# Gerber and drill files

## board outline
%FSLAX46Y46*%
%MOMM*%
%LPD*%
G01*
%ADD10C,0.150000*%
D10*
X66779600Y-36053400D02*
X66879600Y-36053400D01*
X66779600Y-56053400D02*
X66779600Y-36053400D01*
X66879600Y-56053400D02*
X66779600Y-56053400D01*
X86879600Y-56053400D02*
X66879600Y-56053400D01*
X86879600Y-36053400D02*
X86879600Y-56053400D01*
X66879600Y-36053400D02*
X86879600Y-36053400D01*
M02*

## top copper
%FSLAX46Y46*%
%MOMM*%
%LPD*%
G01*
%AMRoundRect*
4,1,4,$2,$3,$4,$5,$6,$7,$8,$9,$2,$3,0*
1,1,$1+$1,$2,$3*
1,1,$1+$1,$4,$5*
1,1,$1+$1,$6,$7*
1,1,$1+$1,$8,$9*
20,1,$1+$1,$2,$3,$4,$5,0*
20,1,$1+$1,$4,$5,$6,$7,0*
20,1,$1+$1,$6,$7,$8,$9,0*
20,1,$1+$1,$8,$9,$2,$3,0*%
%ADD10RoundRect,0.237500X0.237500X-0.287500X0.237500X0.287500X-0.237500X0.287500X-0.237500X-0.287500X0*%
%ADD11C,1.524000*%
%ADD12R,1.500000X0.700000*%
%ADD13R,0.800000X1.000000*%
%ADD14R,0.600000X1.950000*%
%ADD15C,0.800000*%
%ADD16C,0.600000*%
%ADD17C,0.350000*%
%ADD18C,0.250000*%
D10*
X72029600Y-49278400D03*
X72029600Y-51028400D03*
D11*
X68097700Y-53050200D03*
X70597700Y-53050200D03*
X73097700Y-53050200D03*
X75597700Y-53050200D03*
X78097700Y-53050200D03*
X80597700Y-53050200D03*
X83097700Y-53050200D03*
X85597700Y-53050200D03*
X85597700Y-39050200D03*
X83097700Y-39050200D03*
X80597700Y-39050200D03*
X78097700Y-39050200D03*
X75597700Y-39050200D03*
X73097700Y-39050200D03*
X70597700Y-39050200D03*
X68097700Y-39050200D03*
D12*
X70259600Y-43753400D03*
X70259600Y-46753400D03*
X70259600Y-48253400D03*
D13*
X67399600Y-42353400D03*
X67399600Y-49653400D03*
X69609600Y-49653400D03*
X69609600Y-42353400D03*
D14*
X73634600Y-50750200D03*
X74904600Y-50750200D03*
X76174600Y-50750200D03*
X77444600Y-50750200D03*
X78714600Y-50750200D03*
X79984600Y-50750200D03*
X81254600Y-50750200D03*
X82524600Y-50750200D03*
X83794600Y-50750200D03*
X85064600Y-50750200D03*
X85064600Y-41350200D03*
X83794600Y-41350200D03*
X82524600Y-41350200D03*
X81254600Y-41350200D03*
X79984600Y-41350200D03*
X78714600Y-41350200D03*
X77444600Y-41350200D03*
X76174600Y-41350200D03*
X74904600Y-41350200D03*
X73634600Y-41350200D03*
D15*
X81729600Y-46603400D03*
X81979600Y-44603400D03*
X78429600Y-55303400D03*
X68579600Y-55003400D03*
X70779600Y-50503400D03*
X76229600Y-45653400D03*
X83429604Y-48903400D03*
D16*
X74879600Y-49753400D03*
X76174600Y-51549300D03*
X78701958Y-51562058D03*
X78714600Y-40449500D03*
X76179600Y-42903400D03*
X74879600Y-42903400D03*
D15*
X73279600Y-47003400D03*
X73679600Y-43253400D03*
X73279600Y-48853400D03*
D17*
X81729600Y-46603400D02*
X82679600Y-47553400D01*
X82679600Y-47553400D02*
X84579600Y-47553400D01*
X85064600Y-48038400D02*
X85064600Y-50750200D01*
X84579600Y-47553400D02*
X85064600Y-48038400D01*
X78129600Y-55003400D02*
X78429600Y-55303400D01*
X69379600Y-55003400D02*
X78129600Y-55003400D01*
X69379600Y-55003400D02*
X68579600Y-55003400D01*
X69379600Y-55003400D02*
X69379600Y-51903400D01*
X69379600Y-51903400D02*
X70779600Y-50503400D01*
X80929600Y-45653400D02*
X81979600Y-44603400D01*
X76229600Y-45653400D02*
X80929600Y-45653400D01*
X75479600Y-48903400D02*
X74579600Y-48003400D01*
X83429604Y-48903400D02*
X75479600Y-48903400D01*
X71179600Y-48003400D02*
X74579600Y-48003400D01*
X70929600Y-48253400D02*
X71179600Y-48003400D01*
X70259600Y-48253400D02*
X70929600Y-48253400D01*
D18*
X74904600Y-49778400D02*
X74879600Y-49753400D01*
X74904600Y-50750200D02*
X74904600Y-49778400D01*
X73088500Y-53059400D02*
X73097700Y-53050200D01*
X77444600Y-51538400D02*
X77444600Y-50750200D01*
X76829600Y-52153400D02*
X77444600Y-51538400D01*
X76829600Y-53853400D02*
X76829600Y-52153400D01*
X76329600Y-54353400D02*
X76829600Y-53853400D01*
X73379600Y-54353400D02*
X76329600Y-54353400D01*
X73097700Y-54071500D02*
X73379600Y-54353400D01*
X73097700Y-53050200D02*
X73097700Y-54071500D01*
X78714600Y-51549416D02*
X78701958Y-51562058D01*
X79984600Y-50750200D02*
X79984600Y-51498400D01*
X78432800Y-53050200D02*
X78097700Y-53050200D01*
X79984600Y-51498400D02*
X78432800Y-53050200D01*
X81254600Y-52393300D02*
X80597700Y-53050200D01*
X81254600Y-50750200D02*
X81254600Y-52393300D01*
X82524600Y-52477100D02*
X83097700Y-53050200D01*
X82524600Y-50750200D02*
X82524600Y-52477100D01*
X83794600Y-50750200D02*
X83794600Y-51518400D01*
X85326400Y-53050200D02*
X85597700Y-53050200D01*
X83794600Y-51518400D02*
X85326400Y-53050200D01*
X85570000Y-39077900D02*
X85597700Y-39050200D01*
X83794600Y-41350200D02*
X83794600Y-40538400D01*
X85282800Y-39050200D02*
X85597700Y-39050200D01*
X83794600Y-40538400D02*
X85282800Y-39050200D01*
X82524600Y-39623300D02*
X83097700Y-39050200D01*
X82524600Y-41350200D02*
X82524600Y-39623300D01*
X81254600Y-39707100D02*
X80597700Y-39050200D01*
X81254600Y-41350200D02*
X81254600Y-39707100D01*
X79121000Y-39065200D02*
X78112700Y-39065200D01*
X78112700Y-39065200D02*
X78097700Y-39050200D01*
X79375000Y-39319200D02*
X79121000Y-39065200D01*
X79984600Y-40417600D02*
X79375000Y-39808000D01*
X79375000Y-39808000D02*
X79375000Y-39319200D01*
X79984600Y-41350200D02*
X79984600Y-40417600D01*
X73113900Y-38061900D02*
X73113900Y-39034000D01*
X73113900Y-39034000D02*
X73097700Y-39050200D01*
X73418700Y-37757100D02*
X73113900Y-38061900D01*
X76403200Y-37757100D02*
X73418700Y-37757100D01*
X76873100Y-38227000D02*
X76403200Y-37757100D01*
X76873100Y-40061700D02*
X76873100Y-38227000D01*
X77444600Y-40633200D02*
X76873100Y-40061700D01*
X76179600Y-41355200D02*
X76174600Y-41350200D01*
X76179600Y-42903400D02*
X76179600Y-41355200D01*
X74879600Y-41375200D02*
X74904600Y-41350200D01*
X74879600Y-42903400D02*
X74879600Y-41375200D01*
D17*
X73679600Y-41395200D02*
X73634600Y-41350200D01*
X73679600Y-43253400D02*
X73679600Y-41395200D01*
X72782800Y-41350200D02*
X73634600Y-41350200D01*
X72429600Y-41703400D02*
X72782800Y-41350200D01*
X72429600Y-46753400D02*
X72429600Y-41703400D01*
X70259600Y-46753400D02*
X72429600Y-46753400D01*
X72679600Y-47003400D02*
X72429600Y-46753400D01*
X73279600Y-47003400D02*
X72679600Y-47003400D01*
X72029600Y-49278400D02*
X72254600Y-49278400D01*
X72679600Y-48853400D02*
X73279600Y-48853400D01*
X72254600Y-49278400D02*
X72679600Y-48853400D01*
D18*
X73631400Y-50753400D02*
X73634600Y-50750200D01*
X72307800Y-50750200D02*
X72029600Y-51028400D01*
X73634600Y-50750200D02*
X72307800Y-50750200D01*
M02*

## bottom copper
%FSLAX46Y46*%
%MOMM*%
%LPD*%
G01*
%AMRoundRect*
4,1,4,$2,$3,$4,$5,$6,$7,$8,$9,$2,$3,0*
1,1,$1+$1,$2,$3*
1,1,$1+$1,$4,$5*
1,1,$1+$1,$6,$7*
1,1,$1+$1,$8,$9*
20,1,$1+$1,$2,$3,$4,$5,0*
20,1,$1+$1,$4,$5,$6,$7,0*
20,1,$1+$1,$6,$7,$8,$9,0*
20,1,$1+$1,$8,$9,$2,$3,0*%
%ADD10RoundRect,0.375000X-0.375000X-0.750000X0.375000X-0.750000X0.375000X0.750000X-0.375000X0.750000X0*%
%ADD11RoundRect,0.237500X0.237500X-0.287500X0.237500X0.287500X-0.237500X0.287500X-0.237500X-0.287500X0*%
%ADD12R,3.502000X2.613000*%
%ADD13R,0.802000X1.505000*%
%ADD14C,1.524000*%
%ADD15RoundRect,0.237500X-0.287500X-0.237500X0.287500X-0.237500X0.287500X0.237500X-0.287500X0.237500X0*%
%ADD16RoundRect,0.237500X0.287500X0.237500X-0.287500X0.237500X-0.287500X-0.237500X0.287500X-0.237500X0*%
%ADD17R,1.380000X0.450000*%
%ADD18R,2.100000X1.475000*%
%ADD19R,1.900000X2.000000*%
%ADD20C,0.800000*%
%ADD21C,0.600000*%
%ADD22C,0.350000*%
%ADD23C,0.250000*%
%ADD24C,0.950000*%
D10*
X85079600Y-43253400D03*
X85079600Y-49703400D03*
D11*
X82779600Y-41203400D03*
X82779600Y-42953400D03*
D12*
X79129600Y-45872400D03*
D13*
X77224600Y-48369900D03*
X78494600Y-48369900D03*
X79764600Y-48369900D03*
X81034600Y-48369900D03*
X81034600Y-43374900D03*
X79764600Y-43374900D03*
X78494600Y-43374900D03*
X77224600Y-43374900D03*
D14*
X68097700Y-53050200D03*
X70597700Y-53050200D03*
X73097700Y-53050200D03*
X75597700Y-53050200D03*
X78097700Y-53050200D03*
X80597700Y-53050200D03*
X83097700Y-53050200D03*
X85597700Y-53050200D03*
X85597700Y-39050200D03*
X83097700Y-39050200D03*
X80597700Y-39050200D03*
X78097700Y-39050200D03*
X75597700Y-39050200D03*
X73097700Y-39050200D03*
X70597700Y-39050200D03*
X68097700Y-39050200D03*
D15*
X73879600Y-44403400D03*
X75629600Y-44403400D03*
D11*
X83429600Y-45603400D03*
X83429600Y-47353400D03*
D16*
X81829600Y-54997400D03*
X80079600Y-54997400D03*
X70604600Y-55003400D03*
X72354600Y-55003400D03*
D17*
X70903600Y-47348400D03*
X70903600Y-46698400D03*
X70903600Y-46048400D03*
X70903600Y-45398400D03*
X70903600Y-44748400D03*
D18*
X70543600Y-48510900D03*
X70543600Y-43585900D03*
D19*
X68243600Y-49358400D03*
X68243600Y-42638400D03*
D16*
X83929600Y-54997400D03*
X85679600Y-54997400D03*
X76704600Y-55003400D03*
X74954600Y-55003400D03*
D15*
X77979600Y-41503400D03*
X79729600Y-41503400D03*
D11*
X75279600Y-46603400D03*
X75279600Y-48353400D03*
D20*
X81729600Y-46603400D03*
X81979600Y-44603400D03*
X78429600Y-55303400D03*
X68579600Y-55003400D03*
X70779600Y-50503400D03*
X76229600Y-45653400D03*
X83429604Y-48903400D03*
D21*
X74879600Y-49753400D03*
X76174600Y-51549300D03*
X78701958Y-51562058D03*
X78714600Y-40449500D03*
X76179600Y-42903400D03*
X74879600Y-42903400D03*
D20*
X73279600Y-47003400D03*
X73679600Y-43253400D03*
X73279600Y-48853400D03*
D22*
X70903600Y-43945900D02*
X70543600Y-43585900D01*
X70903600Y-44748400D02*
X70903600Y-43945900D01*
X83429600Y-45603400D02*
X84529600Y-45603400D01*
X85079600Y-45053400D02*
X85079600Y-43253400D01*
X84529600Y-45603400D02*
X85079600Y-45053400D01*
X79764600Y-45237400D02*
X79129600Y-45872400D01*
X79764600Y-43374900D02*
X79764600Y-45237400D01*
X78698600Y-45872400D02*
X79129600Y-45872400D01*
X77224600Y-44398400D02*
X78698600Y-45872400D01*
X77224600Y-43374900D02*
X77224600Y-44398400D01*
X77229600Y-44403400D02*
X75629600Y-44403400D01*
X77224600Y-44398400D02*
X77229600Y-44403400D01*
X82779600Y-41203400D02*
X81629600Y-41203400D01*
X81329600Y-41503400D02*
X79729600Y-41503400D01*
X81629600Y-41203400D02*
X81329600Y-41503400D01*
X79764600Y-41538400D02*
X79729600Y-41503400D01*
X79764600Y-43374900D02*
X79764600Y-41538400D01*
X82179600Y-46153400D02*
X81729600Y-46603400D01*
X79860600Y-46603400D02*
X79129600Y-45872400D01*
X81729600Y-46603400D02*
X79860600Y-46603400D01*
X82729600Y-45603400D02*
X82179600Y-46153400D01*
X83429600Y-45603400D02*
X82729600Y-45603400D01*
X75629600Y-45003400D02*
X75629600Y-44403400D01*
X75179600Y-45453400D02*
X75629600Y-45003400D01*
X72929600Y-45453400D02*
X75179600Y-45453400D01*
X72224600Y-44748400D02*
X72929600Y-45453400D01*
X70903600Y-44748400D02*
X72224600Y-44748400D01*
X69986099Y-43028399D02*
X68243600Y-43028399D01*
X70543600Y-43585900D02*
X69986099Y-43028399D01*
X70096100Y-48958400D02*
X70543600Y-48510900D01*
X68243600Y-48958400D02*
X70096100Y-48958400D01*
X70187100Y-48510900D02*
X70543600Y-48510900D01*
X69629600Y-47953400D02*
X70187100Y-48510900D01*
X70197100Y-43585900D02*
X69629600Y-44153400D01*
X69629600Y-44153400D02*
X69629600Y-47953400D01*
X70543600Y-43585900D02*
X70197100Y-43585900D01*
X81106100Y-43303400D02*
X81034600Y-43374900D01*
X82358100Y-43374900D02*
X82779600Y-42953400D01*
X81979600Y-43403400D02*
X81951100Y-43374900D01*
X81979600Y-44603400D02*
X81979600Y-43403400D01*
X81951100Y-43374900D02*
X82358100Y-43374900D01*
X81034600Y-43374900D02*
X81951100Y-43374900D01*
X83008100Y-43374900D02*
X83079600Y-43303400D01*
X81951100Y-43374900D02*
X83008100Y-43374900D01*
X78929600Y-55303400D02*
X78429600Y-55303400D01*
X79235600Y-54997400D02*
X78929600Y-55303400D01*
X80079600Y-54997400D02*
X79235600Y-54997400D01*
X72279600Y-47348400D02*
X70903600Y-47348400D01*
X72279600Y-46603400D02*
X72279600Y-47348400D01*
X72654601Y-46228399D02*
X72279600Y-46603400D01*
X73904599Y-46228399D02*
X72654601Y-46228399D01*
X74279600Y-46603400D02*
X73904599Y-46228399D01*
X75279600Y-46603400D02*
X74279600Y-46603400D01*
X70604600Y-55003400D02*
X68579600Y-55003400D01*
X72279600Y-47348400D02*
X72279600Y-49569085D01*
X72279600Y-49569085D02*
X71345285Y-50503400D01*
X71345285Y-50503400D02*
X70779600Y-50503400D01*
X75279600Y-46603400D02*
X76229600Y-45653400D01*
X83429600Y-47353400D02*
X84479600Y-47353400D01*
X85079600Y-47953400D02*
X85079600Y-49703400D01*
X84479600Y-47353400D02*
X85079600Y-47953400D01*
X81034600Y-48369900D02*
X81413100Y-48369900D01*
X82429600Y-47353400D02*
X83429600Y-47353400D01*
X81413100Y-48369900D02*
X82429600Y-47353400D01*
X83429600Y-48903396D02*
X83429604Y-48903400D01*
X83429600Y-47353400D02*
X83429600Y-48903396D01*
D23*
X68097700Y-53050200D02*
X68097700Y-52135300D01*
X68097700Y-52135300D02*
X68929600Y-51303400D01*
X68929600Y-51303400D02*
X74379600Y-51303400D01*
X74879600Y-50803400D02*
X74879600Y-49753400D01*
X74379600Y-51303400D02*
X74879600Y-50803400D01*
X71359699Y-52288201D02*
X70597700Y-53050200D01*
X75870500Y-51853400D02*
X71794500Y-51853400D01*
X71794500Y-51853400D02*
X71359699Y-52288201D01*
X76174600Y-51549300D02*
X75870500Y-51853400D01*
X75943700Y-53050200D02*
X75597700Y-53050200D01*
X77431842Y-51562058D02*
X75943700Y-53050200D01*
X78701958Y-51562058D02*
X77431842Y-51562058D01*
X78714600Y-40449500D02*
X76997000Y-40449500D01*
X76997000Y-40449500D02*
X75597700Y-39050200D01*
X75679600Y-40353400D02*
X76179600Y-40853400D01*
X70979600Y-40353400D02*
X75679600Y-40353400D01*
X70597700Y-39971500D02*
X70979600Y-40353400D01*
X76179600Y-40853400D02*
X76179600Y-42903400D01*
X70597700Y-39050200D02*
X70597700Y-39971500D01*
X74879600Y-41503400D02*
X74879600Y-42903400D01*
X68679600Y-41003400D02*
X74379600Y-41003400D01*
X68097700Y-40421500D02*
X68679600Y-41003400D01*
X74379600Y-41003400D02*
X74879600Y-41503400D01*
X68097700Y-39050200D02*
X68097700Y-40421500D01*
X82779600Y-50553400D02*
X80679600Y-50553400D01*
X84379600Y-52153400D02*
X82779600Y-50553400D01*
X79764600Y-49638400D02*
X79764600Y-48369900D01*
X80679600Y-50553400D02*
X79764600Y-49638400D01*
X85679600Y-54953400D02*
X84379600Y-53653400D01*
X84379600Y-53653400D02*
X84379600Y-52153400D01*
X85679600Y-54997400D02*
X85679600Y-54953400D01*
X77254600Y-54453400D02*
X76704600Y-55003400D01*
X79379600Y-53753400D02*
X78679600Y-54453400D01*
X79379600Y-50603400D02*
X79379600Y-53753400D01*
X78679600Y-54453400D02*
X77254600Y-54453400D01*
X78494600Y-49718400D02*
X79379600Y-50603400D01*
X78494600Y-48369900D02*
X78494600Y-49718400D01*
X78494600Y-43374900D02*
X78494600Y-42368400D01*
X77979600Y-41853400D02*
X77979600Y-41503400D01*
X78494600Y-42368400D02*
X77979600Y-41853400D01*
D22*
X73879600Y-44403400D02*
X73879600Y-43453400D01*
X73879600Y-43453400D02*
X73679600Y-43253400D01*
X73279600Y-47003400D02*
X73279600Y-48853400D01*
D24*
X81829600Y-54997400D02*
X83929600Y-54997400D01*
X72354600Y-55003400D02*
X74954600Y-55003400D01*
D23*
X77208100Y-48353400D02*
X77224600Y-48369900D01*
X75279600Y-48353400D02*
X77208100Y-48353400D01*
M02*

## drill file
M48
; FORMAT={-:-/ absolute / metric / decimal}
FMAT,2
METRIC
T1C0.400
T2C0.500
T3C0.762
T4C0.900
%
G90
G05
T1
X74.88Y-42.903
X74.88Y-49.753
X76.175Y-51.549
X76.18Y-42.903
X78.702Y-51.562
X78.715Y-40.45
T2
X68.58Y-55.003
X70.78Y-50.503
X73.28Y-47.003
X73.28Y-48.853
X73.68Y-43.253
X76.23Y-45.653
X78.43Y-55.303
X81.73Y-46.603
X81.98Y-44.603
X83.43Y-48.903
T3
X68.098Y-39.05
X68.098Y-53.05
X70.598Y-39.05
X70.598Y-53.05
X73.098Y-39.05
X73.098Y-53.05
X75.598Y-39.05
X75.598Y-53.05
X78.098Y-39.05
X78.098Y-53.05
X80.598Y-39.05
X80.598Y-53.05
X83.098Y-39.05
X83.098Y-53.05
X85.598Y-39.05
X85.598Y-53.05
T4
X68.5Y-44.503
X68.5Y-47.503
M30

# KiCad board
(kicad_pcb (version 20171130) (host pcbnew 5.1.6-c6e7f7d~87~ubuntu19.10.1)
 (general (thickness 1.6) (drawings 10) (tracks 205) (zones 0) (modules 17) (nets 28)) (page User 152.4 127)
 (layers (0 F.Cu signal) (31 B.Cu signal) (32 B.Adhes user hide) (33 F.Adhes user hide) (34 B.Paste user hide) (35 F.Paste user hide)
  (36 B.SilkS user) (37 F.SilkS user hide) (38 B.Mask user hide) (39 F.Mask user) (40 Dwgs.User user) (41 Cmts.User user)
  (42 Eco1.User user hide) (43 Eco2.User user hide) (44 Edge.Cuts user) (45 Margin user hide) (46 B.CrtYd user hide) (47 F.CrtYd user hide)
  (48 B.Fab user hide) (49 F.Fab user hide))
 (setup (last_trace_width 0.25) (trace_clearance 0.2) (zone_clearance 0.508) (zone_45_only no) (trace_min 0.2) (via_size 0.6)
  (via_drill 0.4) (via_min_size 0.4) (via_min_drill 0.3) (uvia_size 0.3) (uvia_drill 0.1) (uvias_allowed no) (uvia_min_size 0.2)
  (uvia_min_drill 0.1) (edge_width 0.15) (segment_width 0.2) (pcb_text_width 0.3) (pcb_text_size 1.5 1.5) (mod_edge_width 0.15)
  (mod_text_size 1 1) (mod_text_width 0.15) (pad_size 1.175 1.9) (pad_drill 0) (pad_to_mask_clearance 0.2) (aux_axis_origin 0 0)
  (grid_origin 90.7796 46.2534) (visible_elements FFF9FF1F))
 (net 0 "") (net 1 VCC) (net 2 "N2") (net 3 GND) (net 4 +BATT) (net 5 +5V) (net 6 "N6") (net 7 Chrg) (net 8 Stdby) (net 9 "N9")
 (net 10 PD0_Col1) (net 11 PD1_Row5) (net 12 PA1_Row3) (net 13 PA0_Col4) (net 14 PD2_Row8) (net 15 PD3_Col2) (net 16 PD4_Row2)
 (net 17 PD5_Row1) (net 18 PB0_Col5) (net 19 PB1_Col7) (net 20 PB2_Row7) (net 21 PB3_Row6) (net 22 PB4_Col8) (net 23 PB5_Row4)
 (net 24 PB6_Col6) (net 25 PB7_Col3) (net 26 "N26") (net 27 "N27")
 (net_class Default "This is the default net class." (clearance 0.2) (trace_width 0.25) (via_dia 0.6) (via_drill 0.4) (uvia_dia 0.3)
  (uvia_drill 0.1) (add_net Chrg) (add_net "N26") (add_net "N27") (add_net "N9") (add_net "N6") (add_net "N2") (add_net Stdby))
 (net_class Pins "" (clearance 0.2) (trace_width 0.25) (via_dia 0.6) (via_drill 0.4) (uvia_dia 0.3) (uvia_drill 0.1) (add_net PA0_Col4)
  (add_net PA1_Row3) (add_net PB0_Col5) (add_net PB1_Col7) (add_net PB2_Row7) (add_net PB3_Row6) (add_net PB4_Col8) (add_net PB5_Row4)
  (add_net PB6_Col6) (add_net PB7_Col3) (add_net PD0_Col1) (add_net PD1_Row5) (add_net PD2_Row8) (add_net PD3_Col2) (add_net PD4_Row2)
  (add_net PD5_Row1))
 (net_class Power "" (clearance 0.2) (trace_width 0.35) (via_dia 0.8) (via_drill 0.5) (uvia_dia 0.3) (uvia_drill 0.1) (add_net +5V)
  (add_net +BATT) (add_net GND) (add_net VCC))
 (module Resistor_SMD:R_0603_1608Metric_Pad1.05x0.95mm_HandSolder (layer F.Cu) (at 72.0296 50.1534 90)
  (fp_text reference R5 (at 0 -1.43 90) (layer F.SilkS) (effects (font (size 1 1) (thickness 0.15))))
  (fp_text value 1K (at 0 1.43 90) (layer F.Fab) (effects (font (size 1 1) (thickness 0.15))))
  (pad 2 smd roundrect (at 0.875 0 90) (size 1.05 0.95) (layers F.Cu F.Paste F.Mask) (roundrect_rratio 0.25) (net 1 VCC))
  (pad 1 smd roundrect (at -0.875 0 90) (size 1.05 0.95) (layers F.Cu F.Paste F.Mask) (roundrect_rratio 0.25) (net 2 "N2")))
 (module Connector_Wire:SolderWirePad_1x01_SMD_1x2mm (layer B.Cu) (at 85.0796 43.2534)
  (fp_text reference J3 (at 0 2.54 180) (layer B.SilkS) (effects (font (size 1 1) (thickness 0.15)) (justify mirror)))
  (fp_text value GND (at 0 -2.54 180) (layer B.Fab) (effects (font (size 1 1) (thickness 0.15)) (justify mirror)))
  (pad 1 smd roundrect (at 0 0) (size 1.5 2.25) (layers B.Cu B.Paste B.Mask) (roundrect_rratio 0.25) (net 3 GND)))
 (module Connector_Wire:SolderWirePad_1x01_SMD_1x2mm (layer B.Cu) (at 85.0796 49.7034)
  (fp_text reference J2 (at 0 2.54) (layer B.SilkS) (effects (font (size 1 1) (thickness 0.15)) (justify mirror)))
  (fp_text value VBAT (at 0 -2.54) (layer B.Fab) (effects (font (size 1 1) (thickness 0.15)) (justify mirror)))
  (pad 1 smd roundrect (at 0 0) (size 1.5 2.25) (layers B.Cu B.Paste B.Mask) (roundrect_rratio 0.25) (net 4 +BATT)))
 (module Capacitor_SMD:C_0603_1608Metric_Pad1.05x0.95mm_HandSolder (layer B.Cu) (at 82.7796 42.0784 90)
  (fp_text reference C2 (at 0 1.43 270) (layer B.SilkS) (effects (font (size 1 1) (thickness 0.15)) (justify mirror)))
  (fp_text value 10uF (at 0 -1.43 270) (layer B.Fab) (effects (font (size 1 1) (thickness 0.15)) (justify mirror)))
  (pad 2 smd roundrect (at 0.875 0 90) (size 1.05 0.95) (layers B.Cu B.Paste B.Mask) (roundrect_rratio 0.25) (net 3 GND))
  (pad 1 smd roundrect (at -0.875 0 90) (size 1.05 0.95) (layers B.Cu B.Paste B.Mask) (roundrect_rratio 0.25) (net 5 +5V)))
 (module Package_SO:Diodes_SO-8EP (layer B.Cu) (at 79.1296 45.8724 270)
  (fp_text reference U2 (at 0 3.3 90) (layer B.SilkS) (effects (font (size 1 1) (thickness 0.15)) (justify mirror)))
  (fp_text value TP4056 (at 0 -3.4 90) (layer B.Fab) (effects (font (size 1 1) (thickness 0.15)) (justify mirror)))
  (pad 9 smd rect (at 0 0 270) (size 2.613 3.502) (layers B.Cu B.Paste B.Mask) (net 3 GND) (solder_paste_margin_ratio -0.2))
  (pad 8 smd rect (at 2.4975 1.905 270) (size 1.505 0.802) (layers B.Cu B.Paste B.Mask) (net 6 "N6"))
  (pad 7 smd rect (at 2.4975 0.635 270) (size 1.505 0.802) (layers B.Cu B.Paste B.Mask) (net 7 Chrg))
  (pad 6 smd rect (at 2.4975 -0.635 270) (size 1.505 0.802) (layers B.Cu B.Paste B.Mask) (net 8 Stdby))
  (pad 5 smd rect (at 2.4975 -1.905 270) (size 1.505 0.802) (layers B.Cu B.Paste B.Mask) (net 4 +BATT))
  (pad 4 smd rect (at -2.4975 -1.905 270) (size 1.505 0.802) (layers B.Cu B.Paste B.Mask) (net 5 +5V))
  (pad 3 smd rect (at -2.4975 -0.635 270) (size 1.505 0.802) (layers B.Cu B.Paste B.Mask) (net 3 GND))
  (pad 2 smd rect (at -2.4975 0.635 270) (size 1.505 0.802) (layers B.Cu B.Paste B.Mask) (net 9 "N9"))
  (pad 1 smd rect (at -2.4975 1.905 270) (size 1.505 0.802) (layers B.Cu B.Paste B.Mask) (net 3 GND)))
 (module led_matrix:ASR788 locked (layer F.Cu) (at 76.8477 46.0502)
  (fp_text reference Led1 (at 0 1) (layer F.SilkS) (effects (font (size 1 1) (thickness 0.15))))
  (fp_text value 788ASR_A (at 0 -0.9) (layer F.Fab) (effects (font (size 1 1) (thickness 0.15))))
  (pad 1 thru_hole circle (at -8.75 7) (size 1.524 1.524) (drill 0.762) (layers *.Cu *.Mask) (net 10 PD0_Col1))
  (pad 2 thru_hole circle (at -6.25 7) (size 1.524 1.524) (drill 0.762) (layers *.Cu *.Mask) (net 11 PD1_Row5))
  (pad 3 thru_hole circle (at -3.75 7) (size 1.524 1.524) (drill 0.762) (layers *.Cu *.Mask) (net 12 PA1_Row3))
  (pad 4 thru_hole circle (at -1.25 7) (size 1.524 1.524) (drill 0.762) (layers *.Cu *.Mask) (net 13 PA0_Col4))
  (pad 5 thru_hole circle (at 1.25 7) (size 1.524 1.524) (drill 0.762) (layers *.Cu *.Mask) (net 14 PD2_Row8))
  (pad 6 thru_hole circle (at 3.75 7) (size 1.524 1.524) (drill 0.762) (layers *.Cu *.Mask) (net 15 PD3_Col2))
  (pad 7 thru_hole circle (at 6.25 7) (size 1.524 1.524) (drill 0.762) (layers *.Cu *.Mask) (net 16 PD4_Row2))
  (pad 8 thru_hole circle (at 8.75 7) (size 1.524 1.524) (drill 0.762) (layers *.Cu *.Mask) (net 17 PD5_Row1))
  (pad 9 thru_hole circle (at 8.75 -7) (size 1.524 1.524) (drill 0.762) (layers *.Cu *.Mask) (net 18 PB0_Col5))
  (pad 10 thru_hole circle (at 6.25 -7) (size 1.524 1.524) (drill 0.762) (layers *.Cu *.Mask) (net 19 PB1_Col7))
  (pad 11 thru_hole circle (at 3.75 -7) (size 1.524 1.524) (drill 0.762) (layers *.Cu *.Mask) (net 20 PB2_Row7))
  (pad 12 thru_hole circle (at 1.25 -7) (size 1.524 1.524) (drill 0.762) (layers *.Cu *.Mask) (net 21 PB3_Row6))
  (pad 13 thru_hole circle (at -1.25 -7) (size 1.524 1.524) (drill 0.762) (layers *.Cu *.Mask) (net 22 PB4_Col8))
  (pad 14 thru_hole circle (at -3.75 -7) (size 1.524 1.524) (drill 0.762) (layers *.Cu *.Mask) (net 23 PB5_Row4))
  (pad 15 thru_hole circle (at -6.25 -7) (size 1.524 1.524) (drill 0.762) (layers *.Cu *.Mask) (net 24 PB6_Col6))
  (pad 16 thru_hole circle (at -8.75 -7) (size 1.524 1.524) (drill 0.762) (layers *.Cu *.Mask) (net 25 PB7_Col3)))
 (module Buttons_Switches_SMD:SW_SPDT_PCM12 (layer F.Cu) (at 68.8296 46.0034 270)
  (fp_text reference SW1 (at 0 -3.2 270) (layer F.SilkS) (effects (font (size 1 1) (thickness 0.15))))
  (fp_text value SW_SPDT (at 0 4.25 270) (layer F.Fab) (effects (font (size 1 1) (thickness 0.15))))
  (pad "" np_thru_hole circle (at -1.5 0.33 270) (size 0.9 0.9) (drill 0.9) (layers *.Cu *.Mask))
  (pad "" np_thru_hole circle (at 1.5 0.33 270) (size 0.9 0.9) (drill 0.9) (layers *.Cu *.Mask))
  (pad 1 smd rect (at -2.25 -1.43 270) (size 0.7 1.5) (layers F.Cu F.Paste F.Mask))
  (pad 2 smd rect (at 0.75 -1.43 270) (size 0.7 1.5) (layers F.Cu F.Paste F.Mask) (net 1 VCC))
  (pad 3 smd rect (at 2.25 -1.43 270) (size 0.7 1.5) (layers F.Cu F.Paste F.Mask) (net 4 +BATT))
  (pad "" smd rect (at -3.65 1.43 270) (size 1 0.8) (layers F.Cu F.Paste F.Mask))
  (pad "" smd rect (at 3.65 1.43 270) (size 1 0.8) (layers F.Cu F.Paste F.Mask))
  (pad "" smd rect (at 3.65 -0.78 270) (size 1 0.8) (layers F.Cu F.Paste F.Mask))
  (pad "" smd rect (at -3.65 -0.78 270) (size 1 0.8) (layers F.Cu F.Paste F.Mask)))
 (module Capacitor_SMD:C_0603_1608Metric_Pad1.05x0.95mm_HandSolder (layer B.Cu) (at 74.7546 44.4034)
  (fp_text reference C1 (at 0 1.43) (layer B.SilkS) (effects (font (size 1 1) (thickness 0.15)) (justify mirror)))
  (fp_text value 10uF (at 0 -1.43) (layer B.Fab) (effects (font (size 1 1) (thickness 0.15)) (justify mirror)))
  (pad 1 smd roundrect (at -0.875 0) (size 1.05 0.95) (layers B.Cu B.Paste B.Mask) (roundrect_rratio 0.25) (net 1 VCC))
  (pad 2 smd roundrect (at 0.875 0) (size 1.05 0.95) (layers B.Cu B.Paste B.Mask) (roundrect_rratio 0.25) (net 3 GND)))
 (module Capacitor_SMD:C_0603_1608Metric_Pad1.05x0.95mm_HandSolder (layer B.Cu) (at 83.4296 46.4784 90)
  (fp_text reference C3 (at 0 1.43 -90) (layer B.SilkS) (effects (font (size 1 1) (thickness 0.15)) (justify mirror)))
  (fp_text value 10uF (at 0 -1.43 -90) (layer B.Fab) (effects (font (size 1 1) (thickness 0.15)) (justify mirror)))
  (pad 2 smd roundrect (at 0.875 0 90) (size 1.05 0.95) (layers B.Cu B.Paste B.Mask) (roundrect_rratio 0.25) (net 3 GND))
  (pad 1 smd roundrect (at -0.875 0 90) (size 1.05 0.95) (layers B.Cu B.Paste B.Mask) (roundrect_rratio 0.25) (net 4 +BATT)))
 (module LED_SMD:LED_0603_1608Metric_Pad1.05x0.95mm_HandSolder (layer B.Cu) (at 80.9546 54.9974 180)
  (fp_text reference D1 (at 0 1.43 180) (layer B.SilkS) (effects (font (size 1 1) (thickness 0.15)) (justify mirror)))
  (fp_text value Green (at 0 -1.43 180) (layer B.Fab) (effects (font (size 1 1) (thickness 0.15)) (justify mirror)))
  (pad 1 smd roundrect (at -0.875 0 180) (size 1.05 0.95) (layers B.Cu B.Paste B.Mask) (roundrect_rratio 0.25) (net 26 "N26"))
  (pad 2 smd roundrect (at 0.875 0 180) (size 1.05 0.95) (layers B.Cu B.Paste B.Mask) (roundrect_rratio 0.25) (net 5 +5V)))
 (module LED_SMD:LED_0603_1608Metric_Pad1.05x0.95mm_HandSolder (layer B.Cu) (at 71.4796 55.0034 180)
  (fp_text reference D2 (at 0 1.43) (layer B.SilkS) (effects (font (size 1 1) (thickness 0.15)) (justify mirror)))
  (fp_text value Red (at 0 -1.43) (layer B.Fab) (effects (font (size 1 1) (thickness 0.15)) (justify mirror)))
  (pad 2 smd roundrect (at 0.875 0 180) (size 1.05 0.95) (layers B.Cu B.Paste B.Mask) (roundrect_rratio 0.25) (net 5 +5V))
  (pad 1 smd roundrect (at -0.875 0 180) (size 1.05 0.95) (layers B.Cu B.Paste B.Mask) (roundrect_rratio 0.25) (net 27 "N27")))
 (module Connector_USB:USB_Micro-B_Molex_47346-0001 (layer B.Cu) (at 69.4436 46.0484 90)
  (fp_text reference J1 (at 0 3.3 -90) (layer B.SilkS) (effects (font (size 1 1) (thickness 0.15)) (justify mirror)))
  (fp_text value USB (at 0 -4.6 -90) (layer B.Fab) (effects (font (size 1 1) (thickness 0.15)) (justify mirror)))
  (pad 1 smd rect (at -1.3 1.46 90) (size 0.45 1.38) (layers B.Cu B.Paste B.Mask) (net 5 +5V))
  (pad 2 smd rect (at -0.65 1.46 90) (size 0.45 1.38) (layers B.Cu B.Paste B.Mask))
  (pad 3 smd rect (at 0 1.46 90) (size 0.45 1.38) (layers B.Cu B.Paste B.Mask))
  (pad 4 smd rect (at 0.65 1.46 90) (size 0.45 1.38) (layers B.Cu B.Paste B.Mask))
  (pad 5 smd rect (at 1.3 1.46 90) (size 0.45 1.38) (layers B.Cu B.Paste B.Mask) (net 3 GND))
  (pad 6 smd rect (at -2.4625 1.1 90) (size 1.475 2.1) (layers B.Cu B.Paste B.Mask) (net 3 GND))
  (pad 6 smd rect (at 2.4625 1.1 90) (size 1.475 2.1) (layers B.Cu B.Paste B.Mask) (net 3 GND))
  (pad 6 smd rect (at -3.31 -1.2 90) (size 2 1.9) (layers B.Cu B.Paste B.Mask) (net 3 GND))
  (pad 6 smd rect (at 3.41 -1.2 90) (size 2 1.9) (layers B.Cu B.Paste B.Mask) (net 3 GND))
  (pad 6 smd rect (at -0.84 -1.2 90) (size 1.175 1.9) (layers Eco1.User))
  (pad 6 smd rect (at 0.84 -1.2 90) (size 1.175 1.9) (layers Eco1.User)))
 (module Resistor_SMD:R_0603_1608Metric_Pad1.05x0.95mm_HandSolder (layer B.Cu) (at 84.8046 54.9974 180)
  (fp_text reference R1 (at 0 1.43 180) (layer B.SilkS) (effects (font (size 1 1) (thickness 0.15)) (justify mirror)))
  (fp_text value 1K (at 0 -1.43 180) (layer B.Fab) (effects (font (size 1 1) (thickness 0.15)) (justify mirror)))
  (pad 2 smd roundrect (at 0.875 0 180) (size 1.05 0.95) (layers B.Cu B.Paste B.Mask) (roundrect_rratio 0.25) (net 26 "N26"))
  (pad 1 smd roundrect (at -0.875 0 180) (size 1.05 0.95) (layers B.Cu B.Paste B.Mask) (roundrect_rratio 0.25) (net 8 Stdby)))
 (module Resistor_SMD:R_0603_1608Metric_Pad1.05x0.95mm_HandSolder (layer B.Cu) (at 75.8296 55.0034 180)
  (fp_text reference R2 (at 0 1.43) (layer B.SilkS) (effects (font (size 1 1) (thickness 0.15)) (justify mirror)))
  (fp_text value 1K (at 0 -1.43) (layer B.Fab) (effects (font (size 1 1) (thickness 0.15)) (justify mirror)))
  (pad 1 smd roundrect (at -0.875 0 180) (size 1.05 0.95) (layers B.Cu B.Paste B.Mask) (roundrect_rratio 0.25) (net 7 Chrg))
  (pad 2 smd roundrect (at 0.875 0 180) (size 1.05 0.95) (layers B.Cu B.Paste B.Mask) (roundrect_rratio 0.25) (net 27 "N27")))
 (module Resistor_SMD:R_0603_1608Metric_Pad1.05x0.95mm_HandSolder (layer B.Cu) (at 78.8546 41.5034)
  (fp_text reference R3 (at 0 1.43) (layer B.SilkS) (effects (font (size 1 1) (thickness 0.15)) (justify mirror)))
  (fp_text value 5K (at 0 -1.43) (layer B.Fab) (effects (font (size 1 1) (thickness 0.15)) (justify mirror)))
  (pad 1 smd roundrect (at -0.875 0) (size 1.05 0.95) (layers B.Cu B.Paste B.Mask) (roundrect_rratio 0.25) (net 9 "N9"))
  (pad 2 smd roundrect (at 0.875 0) (size 1.05 0.95) (layers B.Cu B.Paste B.Mask) (roundrect_rratio 0.25) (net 3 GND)))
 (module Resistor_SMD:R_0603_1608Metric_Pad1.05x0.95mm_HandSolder (layer B.Cu) (at 75.2796 47.4784 90)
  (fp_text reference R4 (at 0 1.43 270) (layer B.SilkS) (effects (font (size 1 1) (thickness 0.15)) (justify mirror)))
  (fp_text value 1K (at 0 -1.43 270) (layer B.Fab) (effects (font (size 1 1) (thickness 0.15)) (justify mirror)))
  (pad 2 smd roundrect (at 0.875 0 90) (size 1.05 0.95) (layers B.Cu B.Paste B.Mask) (roundrect_rratio 0.25) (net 5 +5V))
  (pad 1 smd roundrect (at -0.875 0 90) (size 1.05 0.95) (layers B.Cu B.Paste B.Mask) (roundrect_rratio 0.25) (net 6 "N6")))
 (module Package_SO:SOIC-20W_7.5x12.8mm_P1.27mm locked (layer F.Cu) (at 79.3496 46.0502 90)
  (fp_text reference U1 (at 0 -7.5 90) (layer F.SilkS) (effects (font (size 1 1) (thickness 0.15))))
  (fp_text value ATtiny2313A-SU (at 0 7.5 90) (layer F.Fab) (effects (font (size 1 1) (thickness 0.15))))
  (pad 1 smd rect (at -4.7 -5.715 90) (size 1.95 0.6) (layers F.Cu F.Paste F.Mask) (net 2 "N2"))
  (pad 2 smd rect (at -4.7 -4.445 90) (size 1.95 0.6) (layers F.Cu F.Paste F.Mask) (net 10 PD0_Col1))
  (pad 3 smd rect (at -4.7 -3.175 90) (size 1.95 0.6) (layers F.Cu F.Paste F.Mask) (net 11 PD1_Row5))
  (pad 4 smd rect (at -4.7 -1.905 90) (size 1.95 0.6) (layers F.Cu F.Paste F.Mask) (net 12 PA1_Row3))
  (pad 5 smd rect (at -4.7 -0.635 90) (size 1.95 0.6) (layers F.Cu F.Paste F.Mask) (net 13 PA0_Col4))
  (pad 6 smd rect (at -4.7 0.635 90) (size 1.95 0.6) (layers F.Cu F.Paste F.Mask) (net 14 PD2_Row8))
  (pad 7 smd rect (at -4.7 1.905 90) (size 1.95 0.6) (layers F.Cu F.Paste F.Mask) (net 15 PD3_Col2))
  (pad 8 smd rect (at -4.7 3.175 90) (size 1.95 0.6) (layers F.Cu F.Paste F.Mask) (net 16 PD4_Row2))
  (pad 9 smd rect (at -4.7 4.445 90) (size 1.95 0.6) (layers F.Cu F.Paste F.Mask) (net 17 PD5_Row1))
  (pad 10 smd rect (at -4.7 5.715 90) (size 1.95 0.6) (layers F.Cu F.Paste F.Mask) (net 3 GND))
  (pad 11 smd rect (at 4.7 5.715 90) (size 1.95 0.6) (layers F.Cu F.Paste F.Mask))
  (pad 12 smd rect (at 4.7 4.445 90) (size 1.95 0.6) (layers F.Cu F.Paste F.Mask) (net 18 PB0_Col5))
  (pad 13 smd rect (at 4.7 3.175 90) (size 1.95 0.6) (layers F.Cu F.Paste F.Mask) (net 19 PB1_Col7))
  (pad 14 smd rect (at 4.7 1.905 90) (size 1.95 0.6) (layers F.Cu F.Paste F.Mask) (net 20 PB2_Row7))
  (pad 15 smd rect (at 4.7 0.635 90) (size 1.95 0.6) (layers F.Cu F.Paste F.Mask) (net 21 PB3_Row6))
  (pad 16 smd rect (at 4.7 -0.635 90) (size 1.95 0.6) (layers F.Cu F.Paste F.Mask) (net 22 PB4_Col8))
  (pad 17 smd rect (at 4.7 -1.905 90) (size 1.95 0.6) (layers F.Cu F.Paste F.Mask) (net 23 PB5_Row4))
  (pad 18 smd rect (at 4.7 -3.175 90) (size 1.95 0.6) (layers F.Cu F.Paste F.Mask) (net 24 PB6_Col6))
  (pad 19 smd rect (at 4.7 -4.445 90) (size 1.95 0.6) (layers F.Cu F.Paste F.Mask) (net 25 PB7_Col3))
  (pad 20 smd rect (at 4.7 -5.715 90) (size 1.95 0.6) (layers F.Cu F.Paste F.Mask) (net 1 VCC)))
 (gr_line (start 66.7796 36.0534) (end 66.8796 36.0534) (layer Edge.Cuts) (width 0.15))
 (gr_line (start 66.7796 56.0534) (end 66.7796 36.0534) (layer Edge.Cuts) (width 0.15))
 (gr_line (start 66.8796 56.0534) (end 66.7796 56.0534) (layer Edge.Cuts) (width 0.15))
 (gr_line (start 86.8796 56.0534) (end 66.8796 56.0534) (layer Edge.Cuts) (width 0.15))
 (gr_line (start 86.8796 36.0534) (end 86.8796 56.0534) (layer Edge.Cuts) (width 0.15))
 (gr_line (start 66.8796 36.0534) (end 86.8796 36.0534) (layer Edge.Cuts) (width 0.15))
 (segment (start 70.9036 43.9459) (end 70.5436 43.5859) (width 0.35) (layer B.Cu) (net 3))
 (segment (start 70.9036 44.7484) (end 70.9036 43.9459) (width 0.35) (layer B.Cu) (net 3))
 (segment (start 83.4296 45.6034) (end 84.5296 45.6034) (width 0.35) (layer B.Cu) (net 3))
 (segment (start 85.0796 45.0534) (end 85.0796 43.2534) (width 0.35) (layer B.Cu) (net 3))
 (segment (start 84.5296 45.6034) (end 85.0796 45.0534) (width 0.35) (layer B.Cu) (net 3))
 (segment (start 79.7646 45.2374) (end 79.1296 45.8724) (width 0.35) (layer B.Cu) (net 3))
 (segment (start 79.7646 43.3749) (end 79.7646 45.2374) (width 0.35) (layer B.Cu) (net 3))
 (segment (start 78.6986 45.8724) (end 79.1296 45.8724) (width 0.35) (layer B.Cu) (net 3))
 (segment (start 77.2246 44.3984) (end 78.6986 45.8724) (width 0.35) (layer B.Cu) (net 3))
 (segment (start 77.2246 43.3749) (end 77.2246 44.3984) (width 0.35) (layer B.Cu) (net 3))
 (segment (start 77.2296 44.4034) (end 75.6296 44.4034) (width 0.35) (layer B.Cu) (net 3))
 (segment (start 77.2246 44.3984) (end 77.2296 44.4034) (width 0.35) (layer B.Cu) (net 3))
 (segment (start 82.7796 41.2034) (end 81.6296 41.2034) (width 0.35) (layer B.Cu) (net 3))
 (segment (start 81.3296 41.5034) (end 79.7296 41.5034) (width 0.35) (layer B.Cu) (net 3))
 (segment (start 81.6296 41.2034) (end 81.3296 41.5034) (width 0.35) (layer B.Cu) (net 3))
 (segment (start 79.7646 41.5384) (end 79.7296 41.5034) (width 0.35) (layer B.Cu) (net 3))
 (segment (start 79.7646 43.3749) (end 79.7646 41.5384) (width 0.35) (layer B.Cu) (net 3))
 (segment (start 82.1796 46.1534) (end 81.7296 46.6034) (width 0.35) (layer B.Cu) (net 3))
 (segment (start 79.8606 46.6034) (end 79.1296 45.8724) (width 0.35) (layer B.Cu) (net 3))
 (segment (start 81.7296 46.6034) (end 79.8606 46.6034) (width 0.35) (layer B.Cu) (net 3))
 (segment (start 82.7296 45.6034) (end 82.1796 46.1534) (width 0.35) (layer B.Cu) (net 3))
 (segment (start 83.4296 45.6034) (end 82.7296 45.6034) (width 0.35) (layer B.Cu) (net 3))
 (segment (start 75.6296 45.0034) (end 75.6296 44.4034) (width 0.35) (layer B.Cu) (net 3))
 (segment (start 75.1796 45.4534) (end 75.6296 45.0034) (width 0.35) (layer B.Cu) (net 3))
 (segment (start 72.9296 45.4534) (end 75.1796 45.4534) (width 0.35) (layer B.Cu) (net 3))
 (segment (start 72.2246 44.7484) (end 72.9296 45.4534) (width 0.35) (layer B.Cu) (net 3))
 (segment (start 70.9036 44.7484) (end 72.2246 44.7484) (width 0.35) (layer B.Cu) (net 3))
 (segment (start 69.986099 43.028399) (end 68.2436 43.028399) (width 0.35) (layer B.Cu) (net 3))
 (segment (start 70.5436 43.5859) (end 69.986099 43.028399) (width 0.35) (layer B.Cu) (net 3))
 (segment (start 70.0961 48.9584) (end 70.5436 48.5109) (width 0.35) (layer B.Cu) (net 3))
 (segment (start 68.2436 48.9584) (end 70.0961 48.9584) (width 0.35) (layer B.Cu) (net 3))
 (segment (start 70.1871 48.5109) (end 70.5436 48.5109) (width 0.35) (layer B.Cu) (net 3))
 (segment (start 69.6296 47.9534) (end 70.1871 48.5109) (width 0.35) (layer B.Cu) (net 3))
 (segment (start 70.1971 43.5859) (end 69.6296 44.1534) (width 0.35) (layer B.Cu) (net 3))
 (segment (start 69.6296 44.1534) (end 69.6296 47.9534) (width 0.35) (layer B.Cu) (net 3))
 (segment (start 70.5436 43.5859) (end 70.1971 43.5859) (width 0.35) (layer B.Cu) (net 3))
 (via (at 81.7296 46.6034) (size 0.8) (drill 0.5) (layers F.Cu B.Cu) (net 3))
 (segment (start 81.7296 46.6034) (end 82.6796 47.5534) (width 0.35) (layer F.Cu) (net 3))
 (segment (start 82.6796 47.5534) (end 84.5796 47.5534) (width 0.35) (layer F.Cu) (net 3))
 (segment (start 85.0646 48.0384) (end 85.0646 50.7502) (width 0.35) (layer F.Cu) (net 3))
 (segment (start 84.5796 47.5534) (end 85.0646 48.0384) (width 0.35) (layer F.Cu) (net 3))
 (segment (start 81.1061 43.3034) (end 81.0346 43.3749) (width 0.35) (layer B.Cu) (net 5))
 (via (at 81.9796 44.6034) (size 0.8) (drill 0.5) (layers F.Cu B.Cu) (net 5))
 (segment (start 82.3581 43.3749) (end 82.7796 42.9534) (width 0.35) (layer B.Cu) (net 5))
 (segment (start 81.9796 43.4034) (end 81.9511 43.3749) (width 0.35) (layer B.Cu) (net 5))
 (segment (start 81.9796 44.6034) (end 81.9796 43.4034) (width 0.35) (layer B.Cu) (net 5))
 (segment (start 81.9511 43.3749) (end 82.3581 43.3749) (width 0.35) (layer B.Cu) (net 5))
 (segment (start 81.0346 43.3749) (end 81.9511 43.3749) (width 0.35) (layer B.Cu) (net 5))
 (segment (start 83.0081 43.3749) (end 83.0796 43.3034) (width 0.35) (layer B.Cu) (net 5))
 (segment (start 81.9511 43.3749) (end 83.0081 43.3749) (width 0.35) (layer B.Cu) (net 5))
 (via (at 78.4296 55.3034) (size 0.8) (drill 0.5) (layers F.Cu B.Cu) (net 5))
 (via (at 68.5796 55.0034) (size 0.8) (drill 0.5) (layers F.Cu B.Cu) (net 5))
 (segment (start 78.9296 55.3034) (end 78.4296 55.3034) (width 0.35) (layer B.Cu) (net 5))
 (segment (start 79.2356 54.9974) (end 78.9296 55.3034) (width 0.35) (layer B.Cu) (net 5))
 (segment (start 80.0796 54.9974) (end 79.2356 54.9974) (width 0.35) (layer B.Cu) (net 5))
 (segment (start 72.2796 47.3484) (end 70.9036 47.3484) (width 0.35) (layer B.Cu) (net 5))
 (segment (start 72.2796 46.6034) (end 72.2796 47.3484) (width 0.35) (layer B.Cu) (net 5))
 (segment (start 72.654601 46.228399) (end 72.2796 46.6034) (width 0.35) (layer B.Cu) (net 5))
 (segment (start 73.904599 46.228399) (end 72.654601 46.228399) (width 0.35) (layer B.Cu) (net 5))
 (segment (start 74.2796 46.6034) (end 73.904599 46.228399) (width 0.35) (layer B.Cu) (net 5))
 (segment (start 75.2796 46.6034) (end 74.2796 46.6034) (width 0.35) (layer B.Cu) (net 5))
 (segment (start 78.1296 55.0034) (end 78.4296 55.3034) (width 0.35) (layer F.Cu) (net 5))
 (segment (start 69.3796 55.0034) (end 78.1296 55.0034) (width 0.35) (layer F.Cu) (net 5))
 (segment (start 70.6046 55.0034) (end 68.5796 55.0034) (width 0.35) (layer B.Cu) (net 5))
 (segment (start 69.3796 55.0034) (end 68.5796 55.0034) (width 0.35) (layer F.Cu) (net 5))
 (via (at 70.7796 50.5034) (size 0.8) (drill 0.5) (layers F.Cu B.Cu) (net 5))
 (segment (start 72.2796 47.3484) (end 72.2796 49.569085) (width 0.35) (layer B.Cu) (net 5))
 (segment (start 72.2796 49.569085) (end 71.345285 50.5034) (width 0.35) (layer B.Cu) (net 5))
 (segment (start 71.345285 50.5034) (end 70.7796 50.5034) (width 0.35) (layer B.Cu) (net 5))
 (segment (start 69.3796 55.0034) (end 69.3796 51.9034) (width 0.35) (layer F.Cu) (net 5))
 (segment (start 69.3796 51.9034) (end 70.7796 50.5034) (width 0.35) (layer F.Cu) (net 5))
 (segment (start 75.2796 46.6034) (end 76.2296 45.6534) (width 0.35) (layer B.Cu) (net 5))
 (via (at 76.2296 45.6534) (size 0.8) (drill 0.5) (layers F.Cu B.Cu) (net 5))
 (segment (start 80.9296 45.6534) (end 81.9796 44.6034) (width 0.35) (layer F.Cu) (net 5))
 (segment (start 76.2296 45.6534) (end 80.9296 45.6534) (width 0.35) (layer F.Cu) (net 5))
 (segment (start 83.4296 47.3534) (end 84.4796 47.3534) (width 0.35) (layer B.Cu) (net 4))
 (segment (start 85.0796 47.9534) (end 85.0796 49.7034) (width 0.35) (layer B.Cu) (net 4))
 (segment (start 84.4796 47.3534) (end 85.0796 47.9534) (width 0.35) (layer B.Cu) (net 4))
 (segment (start 81.0346 48.3699) (end 81.4131 48.3699) (width 0.35) (layer B.Cu) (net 4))
 (segment (start 82.4296 47.3534) (end 83.4296 47.3534) (width 0.35) (layer B.Cu) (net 4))
 (segment (start 81.4131 48.3699) (end 82.4296 47.3534) (width 0.35) (layer B.Cu) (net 4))
 (segment (start 83.4296 48.903396) (end 83.429604 48.9034) (width 0.35) (layer B.Cu) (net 4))
 (segment (start 83.4296 47.3534) (end 83.4296 48.903396) (width 0.35) (layer B.Cu) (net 4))
 (via (at 83.429604 48.9034) (size 0.8) (drill 0.5) (layers F.Cu B.Cu) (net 4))
 (segment (start 75.4796 48.9034) (end 74.5796 48.0034) (width 0.35) (layer F.Cu) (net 4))
 (segment (start 83.429604 48.9034) (end 75.4796 48.9034) (width 0.35) (layer F.Cu) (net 4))
 (segment (start 71.1796 48.0034) (end 74.5796 48.0034) (width 0.35) (layer F.Cu) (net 4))
 (segment (start 70.9296 48.2534) (end 71.1796 48.0034) (width 0.35) (layer F.Cu) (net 4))
 (segment (start 70.2596 48.2534) (end 70.9296 48.2534) (width 0.35) (layer F.Cu) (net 4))
 (via (at 74.8796 49.7534) (size 0.6) (drill 0.4) (layers F.Cu B.Cu) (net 10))
 (segment (start 74.9046 49.7784) (end 74.8796 49.7534) (width 0.25) (layer F.Cu) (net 10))
 (segment (start 74.9046 50.7502) (end 74.9046 49.7784) (width 0.25) (layer F.Cu) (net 10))
 (segment (start 68.0977 53.0502) (end 68.0977 52.1353) (width 0.25) (layer B.Cu) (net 10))
 (segment (start 68.0977 52.1353) (end 68.9296 51.3034) (width 0.25) (layer B.Cu) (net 10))
 (segment (start 68.9296 51.3034) (end 74.3796 51.3034) (width 0.25) (layer B.Cu) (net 10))
 (segment (start 74.8796 50.8034) (end 74.8796 49.7534) (width 0.25) (layer B.Cu) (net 10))
 (segment (start 74.3796 51.3034) (end 74.8796 50.8034) (width 0.25) (layer B.Cu) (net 10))
 (via (at 76.1746 51.5493) (size 0.6) (drill 0.4) (layers F.Cu B.Cu) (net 11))
 (segment (start 71.359699 52.288201) (end 70.5977 53.0502) (width 0.25) (layer B.Cu) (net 11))
 (segment (start 75.8705 51.8534) (end 71.7945 51.8534) (width 0.25) (layer B.Cu) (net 11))
 (segment (start 71.7945 51.8534) (end 71.359699 52.288201) (width 0.25) (layer B.Cu) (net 11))
 (segment (start 76.1746 51.5493) (end 75.8705 51.8534) (width 0.25) (layer B.Cu) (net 11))
 (segment (start 73.0885 53.0594) (end 73.0977 53.0502) (width 0.25) (layer F.Cu) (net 12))
 (segment (start 77.4446 51.5384) (end 77.4446 50.7502) (width 0.25) (layer F.Cu) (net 12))
 (segment (start 76.8296 52.1534) (end 77.4446 51.5384) (width 0.25) (layer F.Cu) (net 12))
 (segment (start 76.8296 53.8534) (end 76.8296 52.1534) (width 0.25) (layer F.Cu) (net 12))
 (segment (start 76.3296 54.3534) (end 76.8296 53.8534) (width 0.25) (layer F.Cu) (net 12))
 (segment (start 73.3796 54.3534) (end 76.3296 54.3534) (width 0.25) (layer F.Cu) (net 12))
 (segment (start 73.0977 54.0715) (end 73.3796 54.3534) (width 0.25) (layer F.Cu) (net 12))
 (segment (start 73.0977 53.0502) (end 73.0977 54.0715) (width 0.25) (layer F.Cu) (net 12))
 (segment (start 78.7146 51.549416) (end 78.701958 51.562058) (width 0.25) (layer F.Cu) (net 13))
 (via (at 78.701958 51.562058) (size 0.6) (drill 0.4) (layers F.Cu B.Cu) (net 13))
 (segment (start 75.9437 53.0502) (end 75.5977 53.0502) (width 0.25) (layer B.Cu) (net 13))
 (segment (start 77.431842 51.562058) (end 75.9437 53.0502) (width 0.25) (layer B.Cu) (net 13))
 (segment (start 78.701958 51.562058) (end 77.431842 51.562058) (width 0.25) (layer B.Cu) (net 13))
 (segment (start 79.9846 50.7502) (end 79.9846 51.4984) (width 0.25) (layer F.Cu) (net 14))
 (segment (start 78.4328 53.0502) (end 78.0977 53.0502) (width 0.25) (layer F.Cu) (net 14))
 (segment (start 79.9846 51.4984) (end 78.4328 53.0502) (width 0.25) (layer F.Cu) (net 14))
 (segment (start 81.2546 52.3933) (end 80.5977 53.0502) (width 0.25) (layer F.Cu) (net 15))
 (segment (start 81.2546 50.7502) (end 81.2546 52.3933) (width 0.25) (layer F.Cu) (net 15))
 (segment (start 82.5246 52.4771) (end 83.0977 53.0502) (width 0.25) (layer F.Cu) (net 16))
 (segment (start 82.5246 50.7502) (end 82.5246 52.4771) (width 0.25) (layer F.Cu) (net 16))
 (segment (start 83.7946 50.7502) (end 83.7946 51.5184) (width 0.25) (layer F.Cu) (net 17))
 (segment (start 85.3264 53.0502) (end 85.5977 53.0502) (width 0.25) (layer F.Cu) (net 17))
 (segment (start 83.7946 51.5184) (end 85.3264 53.0502) (width 0.25) (layer F.Cu) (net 17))
 (segment (start 85.57 39.0779) (end 85.5977 39.0502) (width 0.25) (layer F.Cu) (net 18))
 (segment (start 83.7946 41.3502) (end 83.7946 40.5384) (width 0.25) (layer F.Cu) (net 18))
 (segment (start 85.2828 39.0502) (end 85.5977 39.0502) (width 0.25) (layer F.Cu) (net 18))
 (segment (start 83.7946 40.5384) (end 85.2828 39.0502) (width 0.25) (layer F.Cu) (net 18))
 (segment (start 82.5246 39.6233) (end 83.0977 39.0502) (width 0.25) (layer F.Cu) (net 19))
 (segment (start 82.5246 41.3502) (end 82.5246 39.6233) (width 0.25) (layer F.Cu) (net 19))
 (segment (start 81.2546 39.7071) (end 80.5977 39.0502) (width 0.25) (layer F.Cu) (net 20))
 (segment (start 81.2546 41.3502) (end 81.2546 39.7071) (width 0.25) (layer F.Cu) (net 20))
 (segment (start 79.121 39.0652) (end 78.1127 39.0652) (width 0.25) (layer F.Cu) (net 21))
 (segment (start 78.1127 39.0652) (end 78.0977 39.0502) (width 0.25) (layer F.Cu) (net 21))
 (segment (start 79.375 39.3192) (end 79.121 39.0652) (width 0.25) (layer F.Cu) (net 21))
 (segment (start 79.9846 40.4176) (end 79.375 39.808) (width 0.25) (layer F.Cu) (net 21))
 (segment (start 79.375 39.808) (end 79.375 39.3192) (width 0.25) (layer F.Cu) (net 21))
 (segment (start 79.9846 41.3502) (end 79.9846 40.4176) (width 0.25) (layer F.Cu) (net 21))
 (via (at 78.7146 40.4495) (size 0.6) (drill 0.4) (layers F.Cu B.Cu) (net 22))
 (segment (start 78.7146 40.4495) (end 76.997 40.4495) (width 0.25) (layer B.Cu) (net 22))
 (segment (start 76.997 40.4495) (end 75.5977 39.0502) (width 0.25) (layer B.Cu) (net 22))
 (segment (start 73.1139 38.0619) (end 73.1139 39.034) (width 0.25) (layer F.Cu) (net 23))
 (segment (start 73.1139 39.034) (end 73.0977 39.0502) (width 0.25) (layer F.Cu) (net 23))
 (segment (start 73.4187 37.7571) (end 73.1139 38.0619) (width 0.25) (layer F.Cu) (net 23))
 (segment (start 76.4032 37.7571) (end 73.4187 37.7571) (width 0.25) (layer F.Cu) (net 23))
 (segment (start 76.8731 38.227) (end 76.4032 37.7571) (width 0.25) (layer F.Cu) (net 23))
 (segment (start 76.8731 40.0617) (end 76.8731 38.227) (width 0.25) (layer F.Cu) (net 23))
 (segment (start 77.4446 40.6332) (end 76.8731 40.0617) (width 0.25) (layer F.Cu) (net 23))
 (via (at 76.1796 42.9034) (size 0.6) (drill 0.4) (layers F.Cu B.Cu) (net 24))
 (segment (start 76.1796 41.3552) (end 76.1746 41.3502) (width 0.25) (layer F.Cu) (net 24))
 (segment (start 76.1796 42.9034) (end 76.1796 41.3552) (width 0.25) (layer F.Cu) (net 24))
 (segment (start 75.6796 40.3534) (end 76.1796 40.8534) (width 0.25) (layer B.Cu) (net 24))
 (segment (start 70.9796 40.3534) (end 75.6796 40.3534) (width 0.25) (layer B.Cu) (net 24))
 (segment (start 70.5977 39.9715) (end 70.9796 40.3534) (width 0.25) (layer B.Cu) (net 24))
 (segment (start 76.1796 40.8534) (end 76.1796 42.9034) (width 0.25) (layer B.Cu) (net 24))
 (segment (start 70.5977 39.0502) (end 70.5977 39.9715) (width 0.25) (layer B.Cu) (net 24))
 (via (at 74.8796 42.9034) (size 0.6) (drill 0.4) (layers F.Cu B.Cu) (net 25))
 (segment (start 74.8796 41.3752) (end 74.9046 41.3502) (width 0.25) (layer F.Cu) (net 25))
 (segment (start 74.8796 42.9034) (end 74.8796 41.3752) (width 0.25) (layer F.Cu) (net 25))
 (segment (start 74.8796 41.5034) (end 74.8796 42.9034) (width 0.25) (layer B.Cu) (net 25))
 (segment (start 68.6796 41.0034) (end 74.3796 41.0034) (width 0.25) (layer B.Cu) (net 25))
 (segment (start 68.0977 40.4215) (end 68.6796 41.0034) (width 0.25) (layer B.Cu) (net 25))
 (segment (start 74.3796 41.0034) (end 74.8796 41.5034) (width 0.25) (layer B.Cu) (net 25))
 (segment (start 68.0977 39.0502) (end 68.0977 40.4215) (width 0.25) (layer B.Cu) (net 25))
 (segment (start 82.7796 50.5534) (end 80.6796 50.5534) (width 0.25) (layer B.Cu) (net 8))
 (segment (start 84.3796 52.1534) (end 82.7796 50.5534) (width 0.25) (layer B.Cu) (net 8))
 (segment (start 79.7646 49.6384) (end 79.7646 48.3699) (width 0.25) (layer B.Cu) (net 8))
 (segment (start 80.6796 50.5534) (end 79.7646 49.6384) (width 0.25) (layer B.Cu) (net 8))
 (segment (start 85.6796 54.9534) (end 84.3796 53.6534) (width 0.25) (layer B.Cu) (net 8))
 (segment (start 84.3796 53.6534) (end 84.3796 52.1534) (width 0.25) (layer B.Cu) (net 8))
 (segment (start 85.6796 54.9974) (end 85.6796 54.9534) (width 0.25) (layer B.Cu) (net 8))
 (segment (start 77.2546 54.4534) (end 76.7046 55.0034) (width 0.25) (layer B.Cu) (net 7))
 (segment (start 79.3796 53.7534) (end 78.6796 54.4534) (width 0.25) (layer B.Cu) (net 7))
 (segment (start 79.3796 50.6034) (end 79.3796 53.7534) (width 0.25) (layer B.Cu) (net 7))
 (segment (start 78.6796 54.4534) (end 77.2546 54.4534) (width 0.25) (layer B.Cu) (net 7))
 (segment (start 78.4946 49.7184) (end 79.3796 50.6034) (width 0.25) (layer B.Cu) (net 7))
 (segment (start 78.4946 48.3699) (end 78.4946 49.7184) (width 0.25) (layer B.Cu) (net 7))
 (segment (start 78.4946 43.3749) (end 78.4946 42.3684) (width 0.25) (layer B.Cu) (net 9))
 (segment (start 77.9796 41.8534) (end 77.9796 41.5034) (width 0.25) (layer B.Cu) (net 9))
 (segment (start 78.4946 42.3684) (end 77.9796 41.8534) (width 0.25) (layer B.Cu) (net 9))
 (via (at 73.2796 47.0034) (size 0.8) (drill 0.5) (layers F.Cu B.Cu) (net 1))
 (segment (start 73.8796 44.4034) (end 73.8796 43.4534) (width 0.35) (layer B.Cu) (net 1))
 (via (at 73.6796 43.2534) (size 0.8) (drill 0.5) (layers F.Cu B.Cu) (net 1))
 (segment (start 73.8796 43.4534) (end 73.6796 43.2534) (width 0.35) (layer B.Cu) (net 1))
 (segment (start 73.6796 41.3952) (end 73.6346 41.3502) (width 0.35) (layer F.Cu) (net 1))
 (segment (start 73.6796 43.2534) (end 73.6796 41.3952) (width 0.35) (layer F.Cu) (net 1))
 (segment (start 72.7828 41.3502) (end 73.6346 41.3502) (width 0.35) (layer F.Cu) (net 1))
 (segment (start 72.4296 41.7034) (end 72.7828 41.3502) (width 0.35) (layer F.Cu) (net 1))
 (segment (start 72.4296 46.7534) (end 72.4296 41.7034) (width 0.35) (layer F.Cu) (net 1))
 (segment (start 70.2596 46.7534) (end 72.4296 46.7534) (width 0.35) (layer F.Cu) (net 1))
 (segment (start 72.6796 47.0034) (end 72.4296 46.7534) (width 0.35) (layer F.Cu) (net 1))
 (segment (start 73.2796 47.0034) (end 72.6796 47.0034) (width 0.35) (layer F.Cu) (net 1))
 (segment (start 73.2796 47.0034) (end 73.2796 48.8534) (width 0.35) (layer B.Cu) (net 1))
 (via (at 73.2796 48.8534) (size 0.8) (drill 0.5) (layers F.Cu B.Cu) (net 1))
 (segment (start 72.0296 49.2784) (end 72.2546 49.2784) (width 0.35) (layer F.Cu) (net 1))
 (segment (start 72.6796 48.8534) (end 73.2796 48.8534) (width 0.35) (layer F.Cu) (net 1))
 (segment (start 72.2546 49.2784) (end 72.6796 48.8534) (width 0.35) (layer F.Cu) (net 1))
 (segment (start 81.8296 54.9974) (end 83.9296 54.9974) (width 0.95) (layer B.Cu) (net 26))
 (segment (start 72.3546 55.0034) (end 74.9546 55.0034) (width 0.95) (layer B.Cu) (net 27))
 (segment (start 73.6314 50.7534) (end 73.6346 50.7502) (width 0.25) (layer F.Cu) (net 2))
 (segment (start 72.3078 50.7502) (end 72.0296 51.0284) (width 0.25) (layer F.Cu) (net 2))
 (segment (start 73.6346 50.7502) (end 72.3078 50.7502) (width 0.25) (layer F.Cu) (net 2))
 (segment (start 77.2081 48.3534) (end 77.2246 48.3699) (width 0.25) (layer B.Cu) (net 6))
 (segment (start 75.2796 48.3534) (end 77.2081 48.3534) (width 0.25) (layer B.Cu) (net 6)))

